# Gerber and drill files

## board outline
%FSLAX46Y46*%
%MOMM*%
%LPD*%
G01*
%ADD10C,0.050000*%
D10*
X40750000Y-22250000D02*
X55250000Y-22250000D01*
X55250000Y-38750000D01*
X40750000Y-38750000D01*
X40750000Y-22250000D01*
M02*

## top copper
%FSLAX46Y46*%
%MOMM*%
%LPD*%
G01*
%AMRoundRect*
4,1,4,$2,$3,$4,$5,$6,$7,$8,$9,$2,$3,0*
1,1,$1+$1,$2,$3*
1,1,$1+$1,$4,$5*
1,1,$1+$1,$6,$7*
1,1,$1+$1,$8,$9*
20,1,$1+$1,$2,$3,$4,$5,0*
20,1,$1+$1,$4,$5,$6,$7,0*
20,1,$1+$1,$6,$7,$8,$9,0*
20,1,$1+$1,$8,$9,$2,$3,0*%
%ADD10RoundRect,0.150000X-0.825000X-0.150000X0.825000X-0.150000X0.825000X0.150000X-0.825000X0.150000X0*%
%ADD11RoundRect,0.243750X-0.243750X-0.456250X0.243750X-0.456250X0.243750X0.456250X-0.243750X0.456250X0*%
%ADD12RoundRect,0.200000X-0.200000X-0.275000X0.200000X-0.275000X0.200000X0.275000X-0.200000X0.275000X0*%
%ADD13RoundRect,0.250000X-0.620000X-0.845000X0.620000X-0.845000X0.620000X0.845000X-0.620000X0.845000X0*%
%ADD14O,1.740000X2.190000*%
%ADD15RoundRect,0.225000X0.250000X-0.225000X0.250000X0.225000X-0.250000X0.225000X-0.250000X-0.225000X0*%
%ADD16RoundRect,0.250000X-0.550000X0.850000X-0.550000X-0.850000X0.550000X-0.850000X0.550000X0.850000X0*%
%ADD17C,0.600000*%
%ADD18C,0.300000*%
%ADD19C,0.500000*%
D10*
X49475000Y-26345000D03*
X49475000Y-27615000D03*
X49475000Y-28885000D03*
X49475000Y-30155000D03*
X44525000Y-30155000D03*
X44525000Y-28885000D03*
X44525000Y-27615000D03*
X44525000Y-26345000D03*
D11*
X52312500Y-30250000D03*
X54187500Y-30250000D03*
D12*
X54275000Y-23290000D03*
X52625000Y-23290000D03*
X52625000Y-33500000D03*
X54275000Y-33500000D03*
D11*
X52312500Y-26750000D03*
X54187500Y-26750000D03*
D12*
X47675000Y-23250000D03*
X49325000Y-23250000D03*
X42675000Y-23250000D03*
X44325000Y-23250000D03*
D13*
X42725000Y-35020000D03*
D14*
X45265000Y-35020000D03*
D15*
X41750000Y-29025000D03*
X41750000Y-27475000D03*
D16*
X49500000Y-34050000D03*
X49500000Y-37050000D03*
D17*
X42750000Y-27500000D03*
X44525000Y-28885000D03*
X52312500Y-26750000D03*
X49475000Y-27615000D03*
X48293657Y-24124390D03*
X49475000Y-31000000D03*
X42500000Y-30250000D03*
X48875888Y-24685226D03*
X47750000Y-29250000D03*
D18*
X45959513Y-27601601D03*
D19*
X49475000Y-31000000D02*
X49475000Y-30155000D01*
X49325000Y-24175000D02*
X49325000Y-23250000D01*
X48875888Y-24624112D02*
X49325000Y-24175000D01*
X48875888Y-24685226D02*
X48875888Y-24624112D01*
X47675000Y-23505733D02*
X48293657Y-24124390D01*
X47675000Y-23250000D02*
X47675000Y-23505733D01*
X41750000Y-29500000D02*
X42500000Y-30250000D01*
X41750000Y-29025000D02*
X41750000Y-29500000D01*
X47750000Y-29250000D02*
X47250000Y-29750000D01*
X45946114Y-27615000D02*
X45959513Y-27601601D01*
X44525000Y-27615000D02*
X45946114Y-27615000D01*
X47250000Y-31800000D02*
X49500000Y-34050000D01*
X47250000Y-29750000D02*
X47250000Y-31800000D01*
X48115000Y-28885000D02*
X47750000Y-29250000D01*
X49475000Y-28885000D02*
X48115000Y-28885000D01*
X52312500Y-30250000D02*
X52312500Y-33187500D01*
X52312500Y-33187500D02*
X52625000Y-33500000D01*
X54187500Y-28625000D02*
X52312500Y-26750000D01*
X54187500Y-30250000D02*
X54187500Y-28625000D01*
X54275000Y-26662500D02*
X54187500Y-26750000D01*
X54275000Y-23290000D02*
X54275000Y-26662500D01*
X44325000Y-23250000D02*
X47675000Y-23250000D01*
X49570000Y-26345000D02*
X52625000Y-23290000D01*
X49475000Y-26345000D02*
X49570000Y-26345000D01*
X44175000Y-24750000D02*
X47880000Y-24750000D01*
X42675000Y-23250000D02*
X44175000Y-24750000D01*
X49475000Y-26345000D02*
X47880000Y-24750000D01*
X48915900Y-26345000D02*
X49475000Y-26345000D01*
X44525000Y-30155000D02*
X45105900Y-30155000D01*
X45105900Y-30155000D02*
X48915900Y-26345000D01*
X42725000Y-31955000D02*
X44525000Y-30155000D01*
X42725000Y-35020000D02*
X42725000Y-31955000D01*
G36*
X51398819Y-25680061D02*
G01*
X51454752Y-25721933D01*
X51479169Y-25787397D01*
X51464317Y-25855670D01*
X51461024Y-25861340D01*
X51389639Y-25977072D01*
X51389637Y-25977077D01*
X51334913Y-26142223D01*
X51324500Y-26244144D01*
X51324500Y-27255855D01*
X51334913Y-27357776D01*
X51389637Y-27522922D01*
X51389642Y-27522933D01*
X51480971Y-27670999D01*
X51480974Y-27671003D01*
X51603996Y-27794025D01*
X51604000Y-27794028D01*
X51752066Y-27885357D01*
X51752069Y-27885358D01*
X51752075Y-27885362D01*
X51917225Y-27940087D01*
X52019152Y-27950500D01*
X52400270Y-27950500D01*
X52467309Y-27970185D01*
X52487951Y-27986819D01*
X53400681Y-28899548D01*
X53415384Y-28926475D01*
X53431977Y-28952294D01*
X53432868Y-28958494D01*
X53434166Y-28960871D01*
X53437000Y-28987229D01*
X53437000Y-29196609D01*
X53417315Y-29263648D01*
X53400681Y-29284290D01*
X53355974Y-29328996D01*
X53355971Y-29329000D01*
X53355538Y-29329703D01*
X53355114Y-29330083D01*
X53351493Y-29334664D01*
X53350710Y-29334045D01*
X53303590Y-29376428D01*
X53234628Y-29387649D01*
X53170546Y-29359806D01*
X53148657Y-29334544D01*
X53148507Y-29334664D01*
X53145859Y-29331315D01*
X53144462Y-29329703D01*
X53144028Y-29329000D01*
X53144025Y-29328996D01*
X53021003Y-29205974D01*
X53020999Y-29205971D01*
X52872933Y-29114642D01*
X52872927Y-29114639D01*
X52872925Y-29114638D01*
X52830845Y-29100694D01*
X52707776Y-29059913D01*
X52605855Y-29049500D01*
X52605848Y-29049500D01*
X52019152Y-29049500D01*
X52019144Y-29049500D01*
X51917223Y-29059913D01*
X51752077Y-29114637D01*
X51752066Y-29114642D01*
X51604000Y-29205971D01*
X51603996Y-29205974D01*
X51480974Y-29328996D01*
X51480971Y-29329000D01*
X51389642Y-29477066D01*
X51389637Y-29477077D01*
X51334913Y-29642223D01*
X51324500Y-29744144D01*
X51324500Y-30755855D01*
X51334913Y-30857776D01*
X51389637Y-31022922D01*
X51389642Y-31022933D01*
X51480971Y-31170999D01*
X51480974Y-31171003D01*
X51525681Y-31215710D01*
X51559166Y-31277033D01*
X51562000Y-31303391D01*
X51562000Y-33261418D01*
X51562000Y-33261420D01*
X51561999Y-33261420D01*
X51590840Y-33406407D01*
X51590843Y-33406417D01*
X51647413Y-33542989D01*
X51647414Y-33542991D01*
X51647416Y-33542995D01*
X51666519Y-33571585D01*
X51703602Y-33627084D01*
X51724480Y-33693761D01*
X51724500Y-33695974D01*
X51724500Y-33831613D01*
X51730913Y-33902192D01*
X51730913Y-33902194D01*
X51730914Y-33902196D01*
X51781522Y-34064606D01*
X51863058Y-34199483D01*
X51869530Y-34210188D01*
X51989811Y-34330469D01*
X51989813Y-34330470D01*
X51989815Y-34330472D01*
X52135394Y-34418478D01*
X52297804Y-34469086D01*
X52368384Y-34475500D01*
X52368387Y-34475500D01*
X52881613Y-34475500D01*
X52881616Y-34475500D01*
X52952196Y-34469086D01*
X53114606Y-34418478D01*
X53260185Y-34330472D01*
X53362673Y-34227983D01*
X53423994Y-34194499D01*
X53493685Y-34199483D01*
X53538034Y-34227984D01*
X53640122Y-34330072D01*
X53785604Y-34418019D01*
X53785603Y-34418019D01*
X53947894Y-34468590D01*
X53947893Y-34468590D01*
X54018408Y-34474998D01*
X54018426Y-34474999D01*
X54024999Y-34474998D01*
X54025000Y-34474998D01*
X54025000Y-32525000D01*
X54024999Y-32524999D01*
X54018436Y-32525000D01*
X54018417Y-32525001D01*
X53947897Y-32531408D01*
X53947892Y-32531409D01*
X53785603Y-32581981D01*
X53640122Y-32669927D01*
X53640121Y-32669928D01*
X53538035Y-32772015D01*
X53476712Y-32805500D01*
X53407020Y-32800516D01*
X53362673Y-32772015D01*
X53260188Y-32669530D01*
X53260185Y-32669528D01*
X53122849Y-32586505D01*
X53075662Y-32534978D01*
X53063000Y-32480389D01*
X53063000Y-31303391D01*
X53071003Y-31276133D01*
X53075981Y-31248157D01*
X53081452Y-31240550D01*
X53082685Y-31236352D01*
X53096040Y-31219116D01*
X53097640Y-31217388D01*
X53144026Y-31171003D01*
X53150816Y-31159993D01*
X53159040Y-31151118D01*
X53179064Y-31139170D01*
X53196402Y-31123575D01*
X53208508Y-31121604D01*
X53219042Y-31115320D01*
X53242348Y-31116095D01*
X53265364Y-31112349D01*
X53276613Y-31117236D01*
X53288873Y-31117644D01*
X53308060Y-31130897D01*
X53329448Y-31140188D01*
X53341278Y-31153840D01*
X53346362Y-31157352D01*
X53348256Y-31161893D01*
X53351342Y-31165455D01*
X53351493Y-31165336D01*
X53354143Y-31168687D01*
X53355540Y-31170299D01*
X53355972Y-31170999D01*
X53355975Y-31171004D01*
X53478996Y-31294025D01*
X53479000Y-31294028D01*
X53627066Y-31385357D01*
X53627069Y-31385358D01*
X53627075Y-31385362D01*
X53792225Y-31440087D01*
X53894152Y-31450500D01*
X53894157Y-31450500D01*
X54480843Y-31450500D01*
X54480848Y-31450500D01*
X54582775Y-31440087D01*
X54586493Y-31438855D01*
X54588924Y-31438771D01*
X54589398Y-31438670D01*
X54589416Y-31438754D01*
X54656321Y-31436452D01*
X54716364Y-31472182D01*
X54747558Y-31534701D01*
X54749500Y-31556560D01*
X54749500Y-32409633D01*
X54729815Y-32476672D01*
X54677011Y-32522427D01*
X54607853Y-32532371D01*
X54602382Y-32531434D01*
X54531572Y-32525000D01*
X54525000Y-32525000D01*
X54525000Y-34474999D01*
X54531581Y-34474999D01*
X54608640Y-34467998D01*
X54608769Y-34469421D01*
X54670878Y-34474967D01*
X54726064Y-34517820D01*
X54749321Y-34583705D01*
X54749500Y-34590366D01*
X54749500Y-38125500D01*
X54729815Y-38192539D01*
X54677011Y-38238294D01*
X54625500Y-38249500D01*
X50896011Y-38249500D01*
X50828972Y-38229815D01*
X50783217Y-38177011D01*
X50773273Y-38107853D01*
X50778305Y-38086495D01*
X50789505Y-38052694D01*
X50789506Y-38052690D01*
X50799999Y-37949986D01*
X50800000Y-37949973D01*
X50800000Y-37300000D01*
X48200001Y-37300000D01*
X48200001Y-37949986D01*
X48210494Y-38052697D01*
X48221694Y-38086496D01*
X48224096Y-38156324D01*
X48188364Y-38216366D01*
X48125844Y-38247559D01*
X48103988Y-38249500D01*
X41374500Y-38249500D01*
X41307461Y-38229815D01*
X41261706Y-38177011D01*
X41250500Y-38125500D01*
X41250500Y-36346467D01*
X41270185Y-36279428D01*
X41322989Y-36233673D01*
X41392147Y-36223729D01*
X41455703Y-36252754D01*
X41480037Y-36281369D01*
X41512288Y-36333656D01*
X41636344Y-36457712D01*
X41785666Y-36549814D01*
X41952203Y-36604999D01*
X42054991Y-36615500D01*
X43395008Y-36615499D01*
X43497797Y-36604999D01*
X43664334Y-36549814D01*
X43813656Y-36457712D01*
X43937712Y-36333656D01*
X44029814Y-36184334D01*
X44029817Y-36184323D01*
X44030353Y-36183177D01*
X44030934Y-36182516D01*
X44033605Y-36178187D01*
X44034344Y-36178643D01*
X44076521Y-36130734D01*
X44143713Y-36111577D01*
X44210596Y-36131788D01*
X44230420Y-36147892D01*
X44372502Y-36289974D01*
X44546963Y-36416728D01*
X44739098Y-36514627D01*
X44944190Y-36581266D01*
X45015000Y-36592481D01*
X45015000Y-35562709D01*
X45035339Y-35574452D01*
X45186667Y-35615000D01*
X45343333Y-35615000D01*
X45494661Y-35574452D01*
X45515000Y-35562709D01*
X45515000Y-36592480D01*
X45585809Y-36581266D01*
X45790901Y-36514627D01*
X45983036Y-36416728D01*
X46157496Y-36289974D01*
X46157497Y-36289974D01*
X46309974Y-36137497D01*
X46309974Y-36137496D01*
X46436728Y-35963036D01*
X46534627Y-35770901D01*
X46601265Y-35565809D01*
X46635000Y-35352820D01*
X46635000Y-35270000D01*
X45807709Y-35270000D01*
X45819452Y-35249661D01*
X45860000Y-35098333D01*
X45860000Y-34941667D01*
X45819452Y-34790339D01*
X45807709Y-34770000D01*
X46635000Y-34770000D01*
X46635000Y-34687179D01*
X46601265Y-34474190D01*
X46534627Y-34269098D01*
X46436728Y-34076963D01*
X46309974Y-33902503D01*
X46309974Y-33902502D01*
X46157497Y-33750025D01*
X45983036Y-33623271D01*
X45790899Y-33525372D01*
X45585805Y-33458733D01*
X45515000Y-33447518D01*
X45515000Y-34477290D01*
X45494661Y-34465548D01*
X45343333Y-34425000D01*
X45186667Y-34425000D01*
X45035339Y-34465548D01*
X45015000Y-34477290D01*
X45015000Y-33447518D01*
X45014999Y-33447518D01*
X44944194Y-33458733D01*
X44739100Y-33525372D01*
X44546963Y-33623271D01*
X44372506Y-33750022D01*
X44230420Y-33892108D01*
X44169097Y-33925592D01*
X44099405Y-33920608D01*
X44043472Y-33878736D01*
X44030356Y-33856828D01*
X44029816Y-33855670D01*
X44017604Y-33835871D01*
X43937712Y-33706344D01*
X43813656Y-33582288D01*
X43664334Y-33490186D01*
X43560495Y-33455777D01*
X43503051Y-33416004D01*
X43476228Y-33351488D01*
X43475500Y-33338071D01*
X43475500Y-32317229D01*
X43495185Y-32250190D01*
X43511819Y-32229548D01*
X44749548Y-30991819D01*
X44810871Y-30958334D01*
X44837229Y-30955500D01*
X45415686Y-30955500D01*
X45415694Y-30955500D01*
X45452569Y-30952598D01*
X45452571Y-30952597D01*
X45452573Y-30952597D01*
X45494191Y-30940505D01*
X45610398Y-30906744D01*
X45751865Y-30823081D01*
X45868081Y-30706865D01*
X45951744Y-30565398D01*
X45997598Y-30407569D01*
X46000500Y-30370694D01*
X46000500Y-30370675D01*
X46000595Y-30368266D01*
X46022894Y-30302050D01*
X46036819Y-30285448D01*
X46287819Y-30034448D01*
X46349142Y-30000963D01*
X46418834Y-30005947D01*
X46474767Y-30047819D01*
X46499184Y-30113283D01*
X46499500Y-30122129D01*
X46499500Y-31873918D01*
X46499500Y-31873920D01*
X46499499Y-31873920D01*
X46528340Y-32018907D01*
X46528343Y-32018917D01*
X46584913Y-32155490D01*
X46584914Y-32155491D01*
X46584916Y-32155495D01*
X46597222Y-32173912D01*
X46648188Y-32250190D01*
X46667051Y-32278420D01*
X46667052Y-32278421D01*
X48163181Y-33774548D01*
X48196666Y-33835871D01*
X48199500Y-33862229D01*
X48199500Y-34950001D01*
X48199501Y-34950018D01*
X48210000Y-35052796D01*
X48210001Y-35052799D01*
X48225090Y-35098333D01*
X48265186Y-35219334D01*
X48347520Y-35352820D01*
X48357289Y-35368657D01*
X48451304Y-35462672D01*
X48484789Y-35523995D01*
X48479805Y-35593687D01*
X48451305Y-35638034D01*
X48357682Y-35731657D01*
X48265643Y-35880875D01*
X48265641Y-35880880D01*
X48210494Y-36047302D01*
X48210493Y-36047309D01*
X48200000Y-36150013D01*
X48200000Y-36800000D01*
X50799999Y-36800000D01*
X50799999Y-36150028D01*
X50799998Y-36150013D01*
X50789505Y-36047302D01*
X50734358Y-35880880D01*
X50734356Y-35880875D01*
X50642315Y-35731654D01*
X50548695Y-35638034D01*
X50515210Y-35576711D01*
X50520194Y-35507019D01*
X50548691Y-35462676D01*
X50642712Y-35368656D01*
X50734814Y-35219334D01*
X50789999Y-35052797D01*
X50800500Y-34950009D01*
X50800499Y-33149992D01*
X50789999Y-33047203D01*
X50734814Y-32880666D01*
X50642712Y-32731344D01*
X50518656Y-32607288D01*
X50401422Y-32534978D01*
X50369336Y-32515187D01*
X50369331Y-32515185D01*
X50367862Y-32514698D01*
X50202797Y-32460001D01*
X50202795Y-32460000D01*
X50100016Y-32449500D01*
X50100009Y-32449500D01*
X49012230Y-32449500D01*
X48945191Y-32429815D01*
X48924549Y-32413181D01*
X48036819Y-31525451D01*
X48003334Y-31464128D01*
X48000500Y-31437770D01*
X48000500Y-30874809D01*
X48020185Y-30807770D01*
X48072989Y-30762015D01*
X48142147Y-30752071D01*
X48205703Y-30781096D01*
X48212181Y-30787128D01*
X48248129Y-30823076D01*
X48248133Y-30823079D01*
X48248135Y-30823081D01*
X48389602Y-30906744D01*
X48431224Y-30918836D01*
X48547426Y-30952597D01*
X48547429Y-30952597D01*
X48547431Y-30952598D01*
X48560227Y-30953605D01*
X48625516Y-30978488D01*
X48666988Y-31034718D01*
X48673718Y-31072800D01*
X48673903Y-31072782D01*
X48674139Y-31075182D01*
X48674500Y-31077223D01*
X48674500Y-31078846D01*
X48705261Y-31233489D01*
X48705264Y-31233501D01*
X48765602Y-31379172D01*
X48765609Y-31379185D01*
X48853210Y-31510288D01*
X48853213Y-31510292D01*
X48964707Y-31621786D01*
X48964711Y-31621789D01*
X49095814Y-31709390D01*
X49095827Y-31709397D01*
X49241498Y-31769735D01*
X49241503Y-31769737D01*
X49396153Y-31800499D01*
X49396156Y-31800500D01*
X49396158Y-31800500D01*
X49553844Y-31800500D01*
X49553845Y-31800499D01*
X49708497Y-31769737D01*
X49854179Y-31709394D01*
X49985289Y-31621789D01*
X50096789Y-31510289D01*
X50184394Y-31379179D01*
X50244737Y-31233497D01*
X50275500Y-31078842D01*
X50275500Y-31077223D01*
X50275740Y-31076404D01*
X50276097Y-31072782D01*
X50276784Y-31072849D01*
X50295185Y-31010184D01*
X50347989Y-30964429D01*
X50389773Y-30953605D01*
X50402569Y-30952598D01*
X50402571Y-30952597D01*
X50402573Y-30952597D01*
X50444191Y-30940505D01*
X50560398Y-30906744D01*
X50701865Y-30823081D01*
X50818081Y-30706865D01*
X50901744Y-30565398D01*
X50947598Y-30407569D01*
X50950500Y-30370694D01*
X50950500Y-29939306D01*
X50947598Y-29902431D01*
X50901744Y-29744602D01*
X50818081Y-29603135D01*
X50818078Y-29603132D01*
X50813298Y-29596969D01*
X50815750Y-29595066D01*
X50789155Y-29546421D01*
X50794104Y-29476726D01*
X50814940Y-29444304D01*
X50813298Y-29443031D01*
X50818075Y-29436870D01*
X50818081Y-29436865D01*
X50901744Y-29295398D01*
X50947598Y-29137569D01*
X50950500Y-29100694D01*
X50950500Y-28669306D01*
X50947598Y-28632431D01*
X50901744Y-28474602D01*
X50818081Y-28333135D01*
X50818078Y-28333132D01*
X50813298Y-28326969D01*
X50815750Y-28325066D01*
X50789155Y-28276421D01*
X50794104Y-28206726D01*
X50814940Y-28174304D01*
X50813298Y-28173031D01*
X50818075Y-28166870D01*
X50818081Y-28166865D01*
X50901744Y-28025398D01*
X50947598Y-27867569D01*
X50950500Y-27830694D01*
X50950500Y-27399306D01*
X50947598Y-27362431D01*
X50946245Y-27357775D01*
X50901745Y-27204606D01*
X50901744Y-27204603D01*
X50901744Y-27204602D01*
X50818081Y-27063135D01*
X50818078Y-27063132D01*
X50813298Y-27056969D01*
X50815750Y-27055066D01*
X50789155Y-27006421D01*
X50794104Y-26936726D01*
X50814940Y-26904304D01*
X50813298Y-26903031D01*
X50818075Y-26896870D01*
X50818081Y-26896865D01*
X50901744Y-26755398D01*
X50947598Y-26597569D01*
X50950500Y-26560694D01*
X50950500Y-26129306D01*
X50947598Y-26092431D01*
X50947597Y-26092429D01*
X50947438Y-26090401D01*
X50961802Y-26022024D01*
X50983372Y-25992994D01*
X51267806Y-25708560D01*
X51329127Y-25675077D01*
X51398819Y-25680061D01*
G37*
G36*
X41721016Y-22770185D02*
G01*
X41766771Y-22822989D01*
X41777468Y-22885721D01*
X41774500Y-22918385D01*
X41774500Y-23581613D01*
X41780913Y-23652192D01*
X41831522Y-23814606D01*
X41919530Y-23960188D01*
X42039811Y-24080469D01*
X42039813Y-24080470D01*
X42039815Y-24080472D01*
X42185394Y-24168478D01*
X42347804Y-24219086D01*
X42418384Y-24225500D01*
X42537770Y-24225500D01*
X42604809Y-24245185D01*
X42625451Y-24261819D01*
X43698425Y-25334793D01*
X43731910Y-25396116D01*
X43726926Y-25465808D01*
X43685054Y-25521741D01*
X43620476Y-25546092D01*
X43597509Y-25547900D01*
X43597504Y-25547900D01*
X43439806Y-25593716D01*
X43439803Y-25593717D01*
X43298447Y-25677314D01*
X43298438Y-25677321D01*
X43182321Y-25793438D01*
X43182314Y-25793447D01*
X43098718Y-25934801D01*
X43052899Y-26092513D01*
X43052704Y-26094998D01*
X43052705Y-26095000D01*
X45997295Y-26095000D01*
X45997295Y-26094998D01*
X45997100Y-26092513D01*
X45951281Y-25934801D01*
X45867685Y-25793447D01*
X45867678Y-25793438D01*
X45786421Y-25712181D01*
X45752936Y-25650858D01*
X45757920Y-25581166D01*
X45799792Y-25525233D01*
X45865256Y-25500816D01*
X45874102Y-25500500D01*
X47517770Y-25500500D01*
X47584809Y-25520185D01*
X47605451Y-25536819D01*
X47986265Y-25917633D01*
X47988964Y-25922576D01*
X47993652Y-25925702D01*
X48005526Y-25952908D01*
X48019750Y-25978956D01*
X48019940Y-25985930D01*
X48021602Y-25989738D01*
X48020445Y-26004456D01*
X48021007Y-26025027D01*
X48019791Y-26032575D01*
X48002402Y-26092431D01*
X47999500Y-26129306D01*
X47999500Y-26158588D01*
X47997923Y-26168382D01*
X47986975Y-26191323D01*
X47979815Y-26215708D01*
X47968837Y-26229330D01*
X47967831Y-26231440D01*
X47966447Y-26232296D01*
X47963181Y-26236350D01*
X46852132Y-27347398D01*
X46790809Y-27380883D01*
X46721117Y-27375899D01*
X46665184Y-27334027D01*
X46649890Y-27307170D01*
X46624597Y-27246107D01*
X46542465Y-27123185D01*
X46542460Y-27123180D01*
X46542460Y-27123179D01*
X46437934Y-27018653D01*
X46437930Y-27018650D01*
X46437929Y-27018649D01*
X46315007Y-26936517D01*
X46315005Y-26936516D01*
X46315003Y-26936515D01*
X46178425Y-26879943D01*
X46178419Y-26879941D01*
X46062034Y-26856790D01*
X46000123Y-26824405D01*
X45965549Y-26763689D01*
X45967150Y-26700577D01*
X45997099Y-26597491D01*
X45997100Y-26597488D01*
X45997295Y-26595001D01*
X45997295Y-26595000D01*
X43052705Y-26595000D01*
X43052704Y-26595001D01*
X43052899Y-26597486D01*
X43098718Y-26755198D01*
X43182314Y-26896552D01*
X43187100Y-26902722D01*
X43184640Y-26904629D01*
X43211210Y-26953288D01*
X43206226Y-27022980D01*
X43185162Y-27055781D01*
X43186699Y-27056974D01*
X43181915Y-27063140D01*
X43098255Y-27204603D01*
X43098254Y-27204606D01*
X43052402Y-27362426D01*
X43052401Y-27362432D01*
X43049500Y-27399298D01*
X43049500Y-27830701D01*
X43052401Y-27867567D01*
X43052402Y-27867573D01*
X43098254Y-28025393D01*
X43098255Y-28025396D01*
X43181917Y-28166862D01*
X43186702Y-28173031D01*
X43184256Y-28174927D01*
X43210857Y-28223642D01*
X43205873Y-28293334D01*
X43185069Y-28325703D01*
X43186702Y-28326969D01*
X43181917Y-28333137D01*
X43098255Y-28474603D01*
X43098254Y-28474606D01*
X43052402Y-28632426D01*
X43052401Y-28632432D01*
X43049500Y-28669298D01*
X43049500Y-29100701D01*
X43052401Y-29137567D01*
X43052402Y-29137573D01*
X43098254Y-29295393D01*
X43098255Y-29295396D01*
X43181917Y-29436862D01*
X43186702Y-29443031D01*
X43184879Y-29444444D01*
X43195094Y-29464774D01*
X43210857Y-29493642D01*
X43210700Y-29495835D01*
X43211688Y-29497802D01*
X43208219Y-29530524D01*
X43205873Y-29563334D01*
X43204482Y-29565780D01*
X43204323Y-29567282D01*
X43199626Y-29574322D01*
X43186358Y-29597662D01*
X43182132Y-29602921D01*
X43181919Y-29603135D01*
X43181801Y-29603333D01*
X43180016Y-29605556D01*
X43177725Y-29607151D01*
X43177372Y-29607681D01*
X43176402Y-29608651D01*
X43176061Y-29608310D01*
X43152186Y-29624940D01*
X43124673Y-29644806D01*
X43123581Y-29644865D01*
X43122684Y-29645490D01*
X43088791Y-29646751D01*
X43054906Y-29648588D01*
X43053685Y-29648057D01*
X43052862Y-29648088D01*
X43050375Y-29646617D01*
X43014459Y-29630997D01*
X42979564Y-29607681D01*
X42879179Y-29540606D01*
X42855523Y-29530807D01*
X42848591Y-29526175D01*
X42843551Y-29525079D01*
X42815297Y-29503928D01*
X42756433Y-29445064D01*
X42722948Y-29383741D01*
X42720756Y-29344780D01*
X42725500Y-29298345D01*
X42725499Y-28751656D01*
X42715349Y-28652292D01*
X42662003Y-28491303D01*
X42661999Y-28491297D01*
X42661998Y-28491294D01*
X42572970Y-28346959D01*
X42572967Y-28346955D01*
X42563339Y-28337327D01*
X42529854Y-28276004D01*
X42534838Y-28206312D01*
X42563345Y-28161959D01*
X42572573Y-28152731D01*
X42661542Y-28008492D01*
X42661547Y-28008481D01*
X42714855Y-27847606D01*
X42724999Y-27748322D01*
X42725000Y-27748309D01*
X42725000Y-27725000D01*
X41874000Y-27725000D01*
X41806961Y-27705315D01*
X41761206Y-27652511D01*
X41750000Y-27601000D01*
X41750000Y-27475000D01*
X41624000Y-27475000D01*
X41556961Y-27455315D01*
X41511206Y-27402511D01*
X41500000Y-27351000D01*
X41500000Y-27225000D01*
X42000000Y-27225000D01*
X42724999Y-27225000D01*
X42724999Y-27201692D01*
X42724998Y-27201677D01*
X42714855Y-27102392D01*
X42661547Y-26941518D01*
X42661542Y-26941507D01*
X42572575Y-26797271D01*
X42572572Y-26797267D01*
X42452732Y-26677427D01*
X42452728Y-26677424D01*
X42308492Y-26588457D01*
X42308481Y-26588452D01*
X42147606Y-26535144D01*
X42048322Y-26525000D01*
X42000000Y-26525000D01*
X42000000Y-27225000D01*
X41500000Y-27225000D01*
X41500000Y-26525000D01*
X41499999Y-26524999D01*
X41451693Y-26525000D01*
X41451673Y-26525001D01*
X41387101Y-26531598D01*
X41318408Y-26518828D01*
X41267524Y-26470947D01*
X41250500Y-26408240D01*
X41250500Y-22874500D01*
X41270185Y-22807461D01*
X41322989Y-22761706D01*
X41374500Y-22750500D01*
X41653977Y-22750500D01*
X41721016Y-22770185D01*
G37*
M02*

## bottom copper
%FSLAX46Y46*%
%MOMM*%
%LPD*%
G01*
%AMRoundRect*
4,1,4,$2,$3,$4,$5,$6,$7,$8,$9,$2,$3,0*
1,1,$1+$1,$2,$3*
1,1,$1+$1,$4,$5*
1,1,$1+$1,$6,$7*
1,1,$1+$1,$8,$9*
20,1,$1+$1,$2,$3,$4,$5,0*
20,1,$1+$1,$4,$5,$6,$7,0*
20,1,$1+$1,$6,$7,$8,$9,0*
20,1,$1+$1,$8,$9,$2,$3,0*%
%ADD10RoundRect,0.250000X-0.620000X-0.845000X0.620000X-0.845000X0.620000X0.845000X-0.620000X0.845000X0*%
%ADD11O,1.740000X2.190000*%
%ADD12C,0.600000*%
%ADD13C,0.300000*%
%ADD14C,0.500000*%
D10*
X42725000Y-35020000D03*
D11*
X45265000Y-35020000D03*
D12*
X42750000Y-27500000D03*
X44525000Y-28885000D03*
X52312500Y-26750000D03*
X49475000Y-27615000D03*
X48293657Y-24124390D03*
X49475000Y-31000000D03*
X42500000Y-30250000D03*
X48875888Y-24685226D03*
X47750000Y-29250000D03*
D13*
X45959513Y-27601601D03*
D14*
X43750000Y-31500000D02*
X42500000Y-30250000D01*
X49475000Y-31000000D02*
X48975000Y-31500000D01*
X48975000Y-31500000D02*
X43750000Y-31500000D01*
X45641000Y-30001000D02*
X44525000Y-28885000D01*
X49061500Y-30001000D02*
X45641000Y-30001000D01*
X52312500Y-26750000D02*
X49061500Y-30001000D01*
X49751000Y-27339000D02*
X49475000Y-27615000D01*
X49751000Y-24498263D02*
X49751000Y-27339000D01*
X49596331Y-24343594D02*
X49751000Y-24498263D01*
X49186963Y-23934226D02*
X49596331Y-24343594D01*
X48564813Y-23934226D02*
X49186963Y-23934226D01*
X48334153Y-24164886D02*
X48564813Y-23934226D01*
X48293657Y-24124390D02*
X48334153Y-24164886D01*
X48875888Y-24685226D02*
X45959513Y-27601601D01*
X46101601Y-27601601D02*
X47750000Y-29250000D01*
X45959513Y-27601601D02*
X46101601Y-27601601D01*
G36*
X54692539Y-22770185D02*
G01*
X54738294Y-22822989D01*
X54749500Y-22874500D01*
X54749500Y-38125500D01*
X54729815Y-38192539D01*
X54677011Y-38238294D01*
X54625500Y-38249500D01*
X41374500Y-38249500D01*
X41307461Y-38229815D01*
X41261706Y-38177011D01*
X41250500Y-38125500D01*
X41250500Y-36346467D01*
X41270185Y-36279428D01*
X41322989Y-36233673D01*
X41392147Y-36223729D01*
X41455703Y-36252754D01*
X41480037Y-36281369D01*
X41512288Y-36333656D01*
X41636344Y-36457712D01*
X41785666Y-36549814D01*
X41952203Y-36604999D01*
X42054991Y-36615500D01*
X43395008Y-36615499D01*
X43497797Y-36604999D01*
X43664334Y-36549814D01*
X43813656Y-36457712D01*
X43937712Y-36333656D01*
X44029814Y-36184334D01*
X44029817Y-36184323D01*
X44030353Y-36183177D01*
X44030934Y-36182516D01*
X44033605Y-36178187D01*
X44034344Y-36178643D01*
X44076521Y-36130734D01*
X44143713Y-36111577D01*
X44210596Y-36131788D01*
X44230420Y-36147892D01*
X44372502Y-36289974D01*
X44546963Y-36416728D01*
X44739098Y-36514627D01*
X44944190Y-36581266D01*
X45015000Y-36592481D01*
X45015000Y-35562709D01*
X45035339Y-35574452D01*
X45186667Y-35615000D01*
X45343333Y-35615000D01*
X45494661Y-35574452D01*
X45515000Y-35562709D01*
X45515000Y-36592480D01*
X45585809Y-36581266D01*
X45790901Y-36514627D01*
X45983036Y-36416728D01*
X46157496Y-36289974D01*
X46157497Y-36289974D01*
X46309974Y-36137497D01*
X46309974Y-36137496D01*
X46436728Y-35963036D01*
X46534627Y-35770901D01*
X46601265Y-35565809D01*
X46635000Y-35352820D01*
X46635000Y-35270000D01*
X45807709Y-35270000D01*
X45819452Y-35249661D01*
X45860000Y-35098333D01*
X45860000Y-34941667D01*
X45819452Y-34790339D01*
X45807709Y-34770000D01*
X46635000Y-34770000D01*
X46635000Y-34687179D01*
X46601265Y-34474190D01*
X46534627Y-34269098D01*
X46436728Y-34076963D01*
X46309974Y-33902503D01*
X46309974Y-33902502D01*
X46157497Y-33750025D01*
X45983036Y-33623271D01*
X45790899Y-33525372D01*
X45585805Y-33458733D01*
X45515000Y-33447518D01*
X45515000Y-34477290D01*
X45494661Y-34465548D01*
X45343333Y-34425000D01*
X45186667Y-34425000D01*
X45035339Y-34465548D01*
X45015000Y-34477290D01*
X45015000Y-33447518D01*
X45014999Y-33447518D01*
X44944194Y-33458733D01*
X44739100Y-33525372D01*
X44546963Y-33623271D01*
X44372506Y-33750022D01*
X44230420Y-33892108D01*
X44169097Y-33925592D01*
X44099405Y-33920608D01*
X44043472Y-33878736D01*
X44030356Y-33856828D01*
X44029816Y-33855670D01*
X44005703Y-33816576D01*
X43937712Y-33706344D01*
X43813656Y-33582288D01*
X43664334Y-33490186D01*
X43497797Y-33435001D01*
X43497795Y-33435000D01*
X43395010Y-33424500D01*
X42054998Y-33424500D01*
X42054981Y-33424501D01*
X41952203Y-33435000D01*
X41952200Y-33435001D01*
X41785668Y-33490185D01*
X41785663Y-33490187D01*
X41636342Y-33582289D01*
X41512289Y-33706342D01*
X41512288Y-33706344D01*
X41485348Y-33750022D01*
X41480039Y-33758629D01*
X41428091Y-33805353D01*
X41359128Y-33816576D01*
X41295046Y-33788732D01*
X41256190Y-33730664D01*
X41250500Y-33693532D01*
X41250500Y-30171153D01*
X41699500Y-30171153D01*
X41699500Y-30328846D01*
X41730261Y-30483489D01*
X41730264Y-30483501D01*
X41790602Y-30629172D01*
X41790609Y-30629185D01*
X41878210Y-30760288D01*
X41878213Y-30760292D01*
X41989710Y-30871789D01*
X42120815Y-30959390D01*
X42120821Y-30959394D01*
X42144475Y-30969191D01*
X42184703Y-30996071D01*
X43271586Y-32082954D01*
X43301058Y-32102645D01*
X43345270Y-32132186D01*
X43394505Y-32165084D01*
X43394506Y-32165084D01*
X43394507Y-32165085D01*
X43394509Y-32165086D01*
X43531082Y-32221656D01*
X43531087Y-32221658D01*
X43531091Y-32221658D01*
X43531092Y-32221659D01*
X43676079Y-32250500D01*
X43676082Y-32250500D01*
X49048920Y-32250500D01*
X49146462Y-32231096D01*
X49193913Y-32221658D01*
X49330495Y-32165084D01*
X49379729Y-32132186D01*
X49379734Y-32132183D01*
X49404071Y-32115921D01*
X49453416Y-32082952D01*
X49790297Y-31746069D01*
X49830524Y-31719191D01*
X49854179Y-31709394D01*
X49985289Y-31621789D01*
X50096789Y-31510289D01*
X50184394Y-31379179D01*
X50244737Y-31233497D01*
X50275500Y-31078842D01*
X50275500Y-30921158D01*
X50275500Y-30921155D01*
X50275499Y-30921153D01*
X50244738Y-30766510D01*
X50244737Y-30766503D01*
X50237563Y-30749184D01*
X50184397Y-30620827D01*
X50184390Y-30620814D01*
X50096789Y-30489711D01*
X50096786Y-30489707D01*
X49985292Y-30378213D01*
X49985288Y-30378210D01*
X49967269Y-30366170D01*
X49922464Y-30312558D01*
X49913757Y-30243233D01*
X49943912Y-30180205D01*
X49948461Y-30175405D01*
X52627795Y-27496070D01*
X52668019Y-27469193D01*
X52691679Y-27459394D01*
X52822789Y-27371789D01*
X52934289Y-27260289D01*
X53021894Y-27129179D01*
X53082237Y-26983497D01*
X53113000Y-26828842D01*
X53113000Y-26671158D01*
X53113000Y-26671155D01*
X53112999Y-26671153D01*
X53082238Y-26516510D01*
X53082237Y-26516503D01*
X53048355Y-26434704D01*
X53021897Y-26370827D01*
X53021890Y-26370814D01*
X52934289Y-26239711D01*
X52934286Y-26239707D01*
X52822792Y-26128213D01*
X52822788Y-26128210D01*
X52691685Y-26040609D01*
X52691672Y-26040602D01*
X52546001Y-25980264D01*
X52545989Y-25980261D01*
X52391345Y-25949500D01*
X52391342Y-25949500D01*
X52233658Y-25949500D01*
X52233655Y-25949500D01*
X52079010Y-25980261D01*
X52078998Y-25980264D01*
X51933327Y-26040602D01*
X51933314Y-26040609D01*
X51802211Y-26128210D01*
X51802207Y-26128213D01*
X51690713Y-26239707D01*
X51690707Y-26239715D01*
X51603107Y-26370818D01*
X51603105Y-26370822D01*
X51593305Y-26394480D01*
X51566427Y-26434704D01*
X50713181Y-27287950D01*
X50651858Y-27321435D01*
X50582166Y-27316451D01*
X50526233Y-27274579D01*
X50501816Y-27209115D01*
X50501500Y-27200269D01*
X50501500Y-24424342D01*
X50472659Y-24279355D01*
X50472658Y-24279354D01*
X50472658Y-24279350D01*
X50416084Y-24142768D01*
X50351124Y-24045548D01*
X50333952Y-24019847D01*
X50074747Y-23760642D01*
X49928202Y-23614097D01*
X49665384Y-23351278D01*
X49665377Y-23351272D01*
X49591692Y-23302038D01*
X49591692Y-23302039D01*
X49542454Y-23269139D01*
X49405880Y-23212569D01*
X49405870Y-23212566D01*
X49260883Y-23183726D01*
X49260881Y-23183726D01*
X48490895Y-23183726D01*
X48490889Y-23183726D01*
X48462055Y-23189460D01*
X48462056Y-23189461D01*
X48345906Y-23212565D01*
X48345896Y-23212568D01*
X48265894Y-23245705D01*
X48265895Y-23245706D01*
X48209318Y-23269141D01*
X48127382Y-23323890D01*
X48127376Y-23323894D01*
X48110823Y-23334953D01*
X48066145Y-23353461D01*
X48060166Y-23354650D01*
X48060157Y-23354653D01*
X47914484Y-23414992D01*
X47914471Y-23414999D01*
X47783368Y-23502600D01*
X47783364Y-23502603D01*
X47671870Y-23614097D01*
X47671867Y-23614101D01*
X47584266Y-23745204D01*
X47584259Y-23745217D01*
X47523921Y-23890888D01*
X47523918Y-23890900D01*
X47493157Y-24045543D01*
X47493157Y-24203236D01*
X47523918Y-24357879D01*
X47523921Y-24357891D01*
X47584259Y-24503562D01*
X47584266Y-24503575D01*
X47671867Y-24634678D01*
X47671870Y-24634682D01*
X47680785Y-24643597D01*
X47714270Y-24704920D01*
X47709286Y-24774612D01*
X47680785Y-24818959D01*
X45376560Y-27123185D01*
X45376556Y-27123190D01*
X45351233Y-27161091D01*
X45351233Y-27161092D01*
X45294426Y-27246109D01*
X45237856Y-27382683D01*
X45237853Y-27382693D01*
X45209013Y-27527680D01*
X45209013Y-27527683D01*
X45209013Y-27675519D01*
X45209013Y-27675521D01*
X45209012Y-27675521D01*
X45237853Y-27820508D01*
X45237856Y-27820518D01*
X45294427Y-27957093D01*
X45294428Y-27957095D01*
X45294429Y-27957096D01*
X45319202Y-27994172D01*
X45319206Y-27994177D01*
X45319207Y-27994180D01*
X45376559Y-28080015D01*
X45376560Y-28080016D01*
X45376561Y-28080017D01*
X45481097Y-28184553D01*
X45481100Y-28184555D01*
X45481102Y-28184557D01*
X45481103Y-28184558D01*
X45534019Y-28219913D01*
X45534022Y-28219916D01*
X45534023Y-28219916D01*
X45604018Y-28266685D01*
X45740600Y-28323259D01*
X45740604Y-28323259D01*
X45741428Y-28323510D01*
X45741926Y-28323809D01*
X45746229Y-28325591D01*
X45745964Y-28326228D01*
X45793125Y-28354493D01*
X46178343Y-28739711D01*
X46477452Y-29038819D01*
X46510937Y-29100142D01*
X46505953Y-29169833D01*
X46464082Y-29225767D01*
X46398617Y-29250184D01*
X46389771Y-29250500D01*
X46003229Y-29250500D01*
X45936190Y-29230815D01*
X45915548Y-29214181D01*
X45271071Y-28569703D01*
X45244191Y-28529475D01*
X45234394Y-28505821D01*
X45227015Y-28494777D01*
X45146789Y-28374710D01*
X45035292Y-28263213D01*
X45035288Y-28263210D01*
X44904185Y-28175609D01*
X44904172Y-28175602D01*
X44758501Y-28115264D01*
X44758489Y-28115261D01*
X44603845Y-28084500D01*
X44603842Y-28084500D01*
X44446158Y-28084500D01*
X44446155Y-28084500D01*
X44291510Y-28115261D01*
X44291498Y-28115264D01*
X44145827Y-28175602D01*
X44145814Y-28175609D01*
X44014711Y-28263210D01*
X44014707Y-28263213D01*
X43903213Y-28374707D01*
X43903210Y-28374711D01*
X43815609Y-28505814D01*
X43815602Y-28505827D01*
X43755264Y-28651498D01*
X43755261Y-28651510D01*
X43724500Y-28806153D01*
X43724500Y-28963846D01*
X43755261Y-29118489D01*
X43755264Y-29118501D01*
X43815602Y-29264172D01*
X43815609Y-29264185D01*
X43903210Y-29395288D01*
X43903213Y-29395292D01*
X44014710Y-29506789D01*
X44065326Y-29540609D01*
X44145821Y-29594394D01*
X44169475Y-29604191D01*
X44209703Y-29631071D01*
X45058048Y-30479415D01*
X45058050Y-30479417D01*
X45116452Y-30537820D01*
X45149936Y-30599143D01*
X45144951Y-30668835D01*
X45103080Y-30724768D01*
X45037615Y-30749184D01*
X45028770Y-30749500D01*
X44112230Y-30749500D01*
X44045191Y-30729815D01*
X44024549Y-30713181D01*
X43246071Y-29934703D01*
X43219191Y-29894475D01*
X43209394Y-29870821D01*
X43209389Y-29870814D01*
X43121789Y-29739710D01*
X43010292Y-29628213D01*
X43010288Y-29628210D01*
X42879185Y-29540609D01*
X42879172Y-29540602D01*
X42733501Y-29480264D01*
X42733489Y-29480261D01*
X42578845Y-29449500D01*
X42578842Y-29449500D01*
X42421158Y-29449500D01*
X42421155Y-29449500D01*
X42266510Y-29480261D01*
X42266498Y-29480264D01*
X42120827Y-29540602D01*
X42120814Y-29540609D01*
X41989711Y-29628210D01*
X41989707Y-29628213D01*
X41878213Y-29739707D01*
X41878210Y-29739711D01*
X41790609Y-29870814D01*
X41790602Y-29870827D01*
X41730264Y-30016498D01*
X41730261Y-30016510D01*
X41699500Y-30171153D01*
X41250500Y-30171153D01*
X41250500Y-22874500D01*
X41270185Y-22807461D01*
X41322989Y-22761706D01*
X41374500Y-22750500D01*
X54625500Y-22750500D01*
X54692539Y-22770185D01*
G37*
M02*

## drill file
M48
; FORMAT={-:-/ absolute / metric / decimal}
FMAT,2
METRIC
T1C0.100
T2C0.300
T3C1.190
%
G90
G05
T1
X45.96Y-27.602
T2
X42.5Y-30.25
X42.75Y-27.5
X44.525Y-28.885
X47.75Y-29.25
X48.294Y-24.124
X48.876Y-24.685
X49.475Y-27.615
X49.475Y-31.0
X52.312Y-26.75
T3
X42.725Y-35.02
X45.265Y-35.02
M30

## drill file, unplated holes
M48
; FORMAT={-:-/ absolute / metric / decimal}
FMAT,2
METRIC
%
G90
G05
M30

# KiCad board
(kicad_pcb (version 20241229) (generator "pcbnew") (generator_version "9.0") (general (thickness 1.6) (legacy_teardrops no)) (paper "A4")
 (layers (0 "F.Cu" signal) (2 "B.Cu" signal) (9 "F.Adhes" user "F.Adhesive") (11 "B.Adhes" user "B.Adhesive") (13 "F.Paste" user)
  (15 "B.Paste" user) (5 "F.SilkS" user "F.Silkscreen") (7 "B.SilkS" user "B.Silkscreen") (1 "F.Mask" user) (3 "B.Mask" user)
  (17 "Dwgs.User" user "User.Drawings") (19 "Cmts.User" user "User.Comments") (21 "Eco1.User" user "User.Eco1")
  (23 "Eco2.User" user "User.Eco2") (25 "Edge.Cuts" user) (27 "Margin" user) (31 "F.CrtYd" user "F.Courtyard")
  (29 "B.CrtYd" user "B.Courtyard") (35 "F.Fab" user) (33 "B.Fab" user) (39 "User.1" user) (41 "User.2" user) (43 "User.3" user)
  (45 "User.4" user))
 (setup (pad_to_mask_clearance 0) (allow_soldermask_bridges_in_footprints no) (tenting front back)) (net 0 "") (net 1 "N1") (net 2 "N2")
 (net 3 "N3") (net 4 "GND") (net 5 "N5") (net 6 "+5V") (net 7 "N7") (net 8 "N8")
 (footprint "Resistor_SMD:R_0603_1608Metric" (layer "F.Cu") (at 48.5 23.25)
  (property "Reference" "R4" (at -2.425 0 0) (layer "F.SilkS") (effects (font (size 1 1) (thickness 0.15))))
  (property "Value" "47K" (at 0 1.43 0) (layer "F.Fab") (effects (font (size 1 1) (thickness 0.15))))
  (pad "1" smd roundrect (at -0.825 0) (size 0.8 0.95) (layers "F.Cu" "F.Mask" "F.Paste") (roundrect_rratio 0.25) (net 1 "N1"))
  (pad "2" smd roundrect (at 0.825 0) (size 0.8 0.95) (layers "F.Cu" "F.Mask" "F.Paste") (roundrect_rratio 0.25) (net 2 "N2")))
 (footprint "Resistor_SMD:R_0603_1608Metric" (layer "F.Cu") (at 53.45 33.5)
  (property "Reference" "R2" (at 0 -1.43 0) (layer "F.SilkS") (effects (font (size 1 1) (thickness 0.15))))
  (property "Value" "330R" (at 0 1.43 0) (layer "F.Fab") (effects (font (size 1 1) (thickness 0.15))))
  (pad "1" smd roundrect (at -0.825 0) (size 0.8 0.95) (layers "F.Cu" "F.Mask" "F.Paste") (roundrect_rratio 0.25) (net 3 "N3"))
  (pad "2" smd roundrect (at 0.825 0) (size 0.8 0.95) (layers "F.Cu" "F.Mask" "F.Paste") (roundrect_rratio 0.25) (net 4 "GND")))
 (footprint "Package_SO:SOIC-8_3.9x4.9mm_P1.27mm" (layer "F.Cu") (at 47 28.25)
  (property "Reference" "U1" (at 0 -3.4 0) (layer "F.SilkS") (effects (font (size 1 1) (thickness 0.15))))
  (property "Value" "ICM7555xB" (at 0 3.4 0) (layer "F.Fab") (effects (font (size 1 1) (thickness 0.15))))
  (pad "1" smd roundrect (at -2.475 -1.905) (size 1.95 0.6) (layers "F.Cu" "F.Mask" "F.Paste") (roundrect_rratio 0.25) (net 4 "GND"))
  (pad "2" smd roundrect (at -2.475 -0.635) (size 1.95 0.6) (layers "F.Cu" "F.Mask" "F.Paste") (roundrect_rratio 0.25) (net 2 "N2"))
  (pad "3" smd roundrect (at -2.475 0.635) (size 1.95 0.6) (layers "F.Cu" "F.Mask" "F.Paste") (roundrect_rratio 0.25) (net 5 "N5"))
  (pad "4" smd roundrect (at -2.475 1.905) (size 1.95 0.6) (layers "F.Cu" "F.Mask" "F.Paste") (roundrect_rratio 0.25) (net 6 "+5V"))
  (pad "5" smd roundrect (at 2.475 1.905) (size 1.95 0.6) (layers "F.Cu" "F.Mask" "F.Paste") (roundrect_rratio 0.25) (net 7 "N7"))
  (pad "6" smd roundrect (at 2.475 0.635) (size 1.95 0.6) (layers "F.Cu" "F.Mask" "F.Paste") (roundrect_rratio 0.25) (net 2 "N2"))
  (pad "7" smd roundrect (at 2.475 -0.635) (size 1.95 0.6) (layers "F.Cu" "F.Mask" "F.Paste") (roundrect_rratio 0.25) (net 1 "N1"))
  (pad "8" smd roundrect (at 2.475 -1.905) (size 1.95 0.6) (layers "F.Cu" "F.Mask" "F.Paste") (roundrect_rratio 0.25) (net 6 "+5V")))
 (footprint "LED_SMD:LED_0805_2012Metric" (layer "F.Cu") (at 53.25 26.75)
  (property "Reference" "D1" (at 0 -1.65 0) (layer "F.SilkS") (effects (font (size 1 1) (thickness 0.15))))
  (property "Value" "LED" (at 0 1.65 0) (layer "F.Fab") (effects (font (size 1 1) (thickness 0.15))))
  (pad "1" smd roundrect (at -0.9375 0) (size 0.975 1.4) (layers "F.Cu" "F.Mask" "F.Paste") (roundrect_rratio 0.25) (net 5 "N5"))
  (pad "2" smd roundrect (at 0.9375 0) (size 0.975 1.4) (layers "F.Cu" "F.Mask" "F.Paste") (roundrect_rratio 0.25) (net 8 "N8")))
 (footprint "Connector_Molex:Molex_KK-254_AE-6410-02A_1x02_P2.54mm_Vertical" (layer "F.Cu") (at 42.725 35.02)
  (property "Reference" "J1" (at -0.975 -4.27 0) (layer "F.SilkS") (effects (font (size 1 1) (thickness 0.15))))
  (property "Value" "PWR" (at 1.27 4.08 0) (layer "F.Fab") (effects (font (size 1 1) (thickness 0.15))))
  (pad "1" thru_hole roundrect (at 0 0) (size 1.74 2.19) (drill 1.19) (layers "*.Cu" "*.Mask") (remove_unused_layers no)
   (roundrect_rratio 0.143678) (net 6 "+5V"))
  (pad "2" thru_hole oval (at 2.54 0) (size 1.74 2.19) (drill 1.19) (layers "*.Cu" "*.Mask") (remove_unused_layers no) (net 4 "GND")))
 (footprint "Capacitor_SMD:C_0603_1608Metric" (layer "F.Cu") (at 41.75 28.25 90)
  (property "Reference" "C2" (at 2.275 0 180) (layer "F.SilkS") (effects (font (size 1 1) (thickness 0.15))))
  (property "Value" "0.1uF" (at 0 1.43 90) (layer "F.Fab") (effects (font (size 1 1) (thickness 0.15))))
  (pad "1" smd roundrect (at -0.775 0 90) (size 0.9 0.95) (layers "F.Cu" "F.Mask" "F.Paste") (roundrect_rratio 0.25) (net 7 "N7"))
  (pad "2" smd roundrect (at 0.775 0 90) (size 0.9 0.95) (layers "F.Cu" "F.Mask" "F.Paste") (roundrect_rratio 0.25) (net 4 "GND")))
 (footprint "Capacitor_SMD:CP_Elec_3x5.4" (layer "F.Cu") (at 49.5 35.55 -90)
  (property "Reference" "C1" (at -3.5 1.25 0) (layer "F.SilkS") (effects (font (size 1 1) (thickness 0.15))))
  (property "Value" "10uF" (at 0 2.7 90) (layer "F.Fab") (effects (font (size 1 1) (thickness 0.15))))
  (pad "1" smd roundrect (at -1.5 0 270) (size 2.2 1.6) (layers "F.Cu" "F.Mask" "F.Paste") (roundrect_rratio 0.15625) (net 2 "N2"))
  (pad "2" smd roundrect (at 1.5 0 270) (size 2.2 1.6) (layers "F.Cu" "F.Mask" "F.Paste") (roundrect_rratio 0.15625) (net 4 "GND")))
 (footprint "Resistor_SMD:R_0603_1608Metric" (layer "F.Cu") (at 43.5 23.25)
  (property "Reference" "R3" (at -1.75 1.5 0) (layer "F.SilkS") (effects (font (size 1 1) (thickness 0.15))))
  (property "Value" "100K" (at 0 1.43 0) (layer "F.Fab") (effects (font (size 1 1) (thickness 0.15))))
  (pad "1" smd roundrect (at -0.825 0) (size 0.8 0.95) (layers "F.Cu" "F.Mask" "F.Paste") (roundrect_rratio 0.25) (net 6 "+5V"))
  (pad "2" smd roundrect (at 0.825 0) (size 0.8 0.95) (layers "F.Cu" "F.Mask" "F.Paste") (roundrect_rratio 0.25) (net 1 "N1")))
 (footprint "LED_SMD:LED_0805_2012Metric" (layer "F.Cu") (at 53.25 30.25)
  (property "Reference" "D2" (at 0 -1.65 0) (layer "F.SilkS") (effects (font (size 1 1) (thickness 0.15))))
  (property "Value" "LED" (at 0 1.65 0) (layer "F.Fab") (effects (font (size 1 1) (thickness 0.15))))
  (pad "1" smd roundrect (at -0.9375 0) (size 0.975 1.4) (layers "F.Cu" "F.Mask" "F.Paste") (roundrect_rratio 0.25) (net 3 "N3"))
  (pad "2" smd roundrect (at 0.9375 0) (size 0.975 1.4) (layers "F.Cu" "F.Mask" "F.Paste") (roundrect_rratio 0.25) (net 5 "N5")))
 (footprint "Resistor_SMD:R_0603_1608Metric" (layer "F.Cu") (at 53.45 23.29)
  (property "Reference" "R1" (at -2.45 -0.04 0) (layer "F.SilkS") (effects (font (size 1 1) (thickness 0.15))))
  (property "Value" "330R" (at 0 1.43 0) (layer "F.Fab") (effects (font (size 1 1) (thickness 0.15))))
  (pad "1" smd roundrect (at -0.825 0) (size 0.8 0.95) (layers "F.Cu" "F.Mask" "F.Paste") (roundrect_rratio 0.25) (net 6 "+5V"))
  (pad "2" smd roundrect (at 0.825 0) (size 0.8 0.95) (layers "F.Cu" "F.Mask" "F.Paste") (roundrect_rratio 0.25) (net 8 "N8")))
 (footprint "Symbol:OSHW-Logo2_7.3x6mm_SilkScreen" (layer "B.Cu") (at 50.264684 27 180)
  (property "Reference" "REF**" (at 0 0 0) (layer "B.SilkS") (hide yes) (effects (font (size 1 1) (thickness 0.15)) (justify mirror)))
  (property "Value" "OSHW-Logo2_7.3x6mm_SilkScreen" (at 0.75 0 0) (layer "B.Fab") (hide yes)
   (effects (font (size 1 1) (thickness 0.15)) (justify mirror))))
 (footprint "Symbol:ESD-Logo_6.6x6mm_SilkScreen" (layer "B.Cu") (at 50.014684 33.75 180)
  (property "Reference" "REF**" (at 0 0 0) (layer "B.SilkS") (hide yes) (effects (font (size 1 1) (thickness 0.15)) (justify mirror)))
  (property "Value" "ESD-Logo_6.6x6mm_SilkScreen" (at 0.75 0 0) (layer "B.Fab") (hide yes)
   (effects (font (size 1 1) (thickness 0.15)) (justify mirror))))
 (gr_rect (start 40.75 22.25) (end 55.25 38.75) (stroke (width 0.05) (type default)) (fill no) (layer "Edge.Cuts"))
 (via (at 42.75 27.5) (size 0.6) (drill 0.3) (layers "F.Cu" "B.Cu") (free yes) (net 4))
 (segment (start 48.875888 24.624112) (end 49.325 24.175) (width 0.5) (layer "F.Cu") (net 2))
 (segment (start 44.525 27.615) (end 45.946114 27.615) (width 0.5) (layer "F.Cu") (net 2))
 (segment (start 48.115 28.885) (end 47.75 29.25) (width 0.5) (layer "F.Cu") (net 2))
 (segment (start 45.946114 27.615) (end 45.959513 27.601601) (width 0.5) (layer "F.Cu") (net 2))
 (segment (start 47.75 29.25) (end 47.25 29.75) (width 0.5) (layer "F.Cu") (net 2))
 (segment (start 48.875888 24.685226) (end 48.875888 24.624112) (width 0.5) (layer "F.Cu") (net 2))
 (segment (start 49.475 28.885) (end 48.115 28.885) (width 0.5) (layer "F.Cu") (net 2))
 (segment (start 47.25 29.75) (end 47.25 31.8) (width 0.5) (layer "F.Cu") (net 2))
 (segment (start 47.25 31.8) (end 49.5 34.05) (width 0.5) (layer "F.Cu") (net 2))
 (segment (start 49.325 24.175) (end 49.325 23.25) (width 0.5) (layer "F.Cu") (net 2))
 (via (at 47.75 29.25) (size 0.6) (drill 0.3) (layers "F.Cu" "B.Cu") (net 2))
 (via (at 48.875888 24.685226) (size 0.6) (drill 0.3) (layers "F.Cu" "B.Cu") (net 2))
 (via micro (at 45.959513 27.601601) (size 0.3) (drill 0.1) (layers "F.Cu" "B.Cu") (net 2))
 (segment (start 45.959513 27.601601) (end 46.101601 27.601601) (width 0.5) (layer "B.Cu") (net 2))
 (segment (start 48.875888 24.685226) (end 45.959513 27.601601) (width 0.5) (layer "B.Cu") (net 2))
 (segment (start 46.101601 27.601601) (end 47.75 29.25) (width 0.5) (layer "B.Cu") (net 2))
 (segment (start 49.475 31) (end 49.475 30.155) (width 0.5) (layer "F.Cu") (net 7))
 (segment (start 41.75 29.025) (end 41.75 29.5) (width 0.5) (layer "F.Cu") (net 7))
 (segment (start 41.75 29.5) (end 42.5 30.25) (width 0.5) (layer "F.Cu") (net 7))
 (via (at 49.475 31) (size 0.6) (drill 0.3) (layers "F.Cu" "B.Cu") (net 7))
 (via (at 42.5 30.25) (size 0.6) (drill 0.3) (layers "F.Cu" "B.Cu") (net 7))
 (segment (start 48.975 31.5) (end 43.75 31.5) (width 0.5) (layer "B.Cu") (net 7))
 (segment (start 49.475 31) (end 48.975 31.5) (width 0.5) (layer "B.Cu") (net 7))
 (segment (start 43.75 31.5) (end 42.5 30.25) (width 0.5) (layer "B.Cu") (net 7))
 (segment (start 54.275 23.29) (end 54.275 26.6625) (width 0.5) (layer "F.Cu") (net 8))
 (segment (start 54.275 26.6625) (end 54.1875 26.75) (width 0.5) (layer "F.Cu") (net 8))
 (segment (start 54.1875 30.25) (end 54.1875 28.625) (width 0.5) (layer "F.Cu") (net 5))
 (segment (start 54.1875 28.625) (end 52.3125 26.75) (width 0.5) (layer "F.Cu") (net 5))
 (via (at 44.525 28.885) (size 0.6) (drill 0.3) (layers "F.Cu" "B.Cu") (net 5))
 (via (at 52.3125 26.75) (size 0.6) (drill 0.3) (layers "F.Cu" "B.Cu") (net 5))
 (segment (start 52.3125 26.75) (end 49.0615 30.001) (width 0.5) (layer "B.Cu") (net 5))
 (segment (start 45.641 30.001) (end 44.525 28.885) (width 0.5) (layer "B.Cu") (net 5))
 (segment (start 49.0615 30.001) (end 45.641 30.001) (width 0.5) (layer "B.Cu") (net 5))
 (segment (start 52.3125 30.25) (end 52.3125 33.1875) (width 0.5) (layer "F.Cu") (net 3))
 (segment (start 52.3125 33.1875) (end 52.625 33.5) (width 0.5) (layer "F.Cu") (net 3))
 (segment (start 49.475 26.345) (end 49.57 26.345) (width 0.5) (layer "F.Cu") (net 6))
 (segment (start 48.9159 26.345) (end 49.475 26.345) (width 0.5) (layer "F.Cu") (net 6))
 (segment (start 42.675 23.25) (end 44.175 24.75) (width 0.5) (layer "F.Cu") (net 6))
 (segment (start 49.475 26.345) (end 47.88 24.75) (width 0.5) (layer "F.Cu") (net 6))
 (segment (start 42.725 31.955) (end 44.525 30.155) (width 0.5) (layer "F.Cu") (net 6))
 (segment (start 44.525 30.155) (end 45.1059 30.155) (width 0.5) (layer "F.Cu") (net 6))
 (segment (start 42.725 35.02) (end 42.725 31.955) (width 0.5) (layer "F.Cu") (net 6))
 (segment (start 49.57 26.345) (end 52.625 23.29) (width 0.5) (layer "F.Cu") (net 6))
 (segment (start 45.1059 30.155) (end 48.9159 26.345) (width 0.5) (layer "F.Cu") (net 6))
 (segment (start 44.175 24.75) (end 47.88 24.75) (width 0.5) (layer "F.Cu") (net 6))
 (segment (start 44.325 23.25) (end 47.675 23.25) (width 0.5) (layer "F.Cu") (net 1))
 (segment (start 47.675 23.25) (end 47.675 23.505733) (width 0.5) (layer "F.Cu") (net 1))
 (segment (start 47.675 23.505733) (end 48.293657 24.12439) (width 0.5) (layer "F.Cu") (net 1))
 (via (at 49.475 27.615) (size 0.6) (drill 0.3) (layers "F.Cu" "B.Cu") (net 1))
 (via (at 48.293657 24.12439) (size 0.6) (drill 0.3) (layers "F.Cu" "B.Cu") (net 1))
 (segment (start 49.751 27.339) (end 49.475 27.615) (width 0.5) (layer "B.Cu") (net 1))
 (segment (start 49.596331 24.343594) (end 49.751 24.498263) (width 0.5) (layer "B.Cu") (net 1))
 (segment (start 48.293657 24.12439) (end 48.334153 24.164886) (width 0.5) (layer "B.Cu") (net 1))
 (segment (start 48.334153 24.164886) (end 48.564813 23.934226) (width 0.5) (layer "B.Cu") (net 1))
 (segment (start 48.564813 23.934226) (end 49.186963 23.934226) (width 0.5) (layer "B.Cu") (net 1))
 (segment (start 49.751 24.498263) (end 49.751 27.339) (width 0.5) (layer "B.Cu") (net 1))
 (segment (start 49.186963 23.934226) (end 49.596331 24.343594) (width 0.5) (layer "B.Cu") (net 1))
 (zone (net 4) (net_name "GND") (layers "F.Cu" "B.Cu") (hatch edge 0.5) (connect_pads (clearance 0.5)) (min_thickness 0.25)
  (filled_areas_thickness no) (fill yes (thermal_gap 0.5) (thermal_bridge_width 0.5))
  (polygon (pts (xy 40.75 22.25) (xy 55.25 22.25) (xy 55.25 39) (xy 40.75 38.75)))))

